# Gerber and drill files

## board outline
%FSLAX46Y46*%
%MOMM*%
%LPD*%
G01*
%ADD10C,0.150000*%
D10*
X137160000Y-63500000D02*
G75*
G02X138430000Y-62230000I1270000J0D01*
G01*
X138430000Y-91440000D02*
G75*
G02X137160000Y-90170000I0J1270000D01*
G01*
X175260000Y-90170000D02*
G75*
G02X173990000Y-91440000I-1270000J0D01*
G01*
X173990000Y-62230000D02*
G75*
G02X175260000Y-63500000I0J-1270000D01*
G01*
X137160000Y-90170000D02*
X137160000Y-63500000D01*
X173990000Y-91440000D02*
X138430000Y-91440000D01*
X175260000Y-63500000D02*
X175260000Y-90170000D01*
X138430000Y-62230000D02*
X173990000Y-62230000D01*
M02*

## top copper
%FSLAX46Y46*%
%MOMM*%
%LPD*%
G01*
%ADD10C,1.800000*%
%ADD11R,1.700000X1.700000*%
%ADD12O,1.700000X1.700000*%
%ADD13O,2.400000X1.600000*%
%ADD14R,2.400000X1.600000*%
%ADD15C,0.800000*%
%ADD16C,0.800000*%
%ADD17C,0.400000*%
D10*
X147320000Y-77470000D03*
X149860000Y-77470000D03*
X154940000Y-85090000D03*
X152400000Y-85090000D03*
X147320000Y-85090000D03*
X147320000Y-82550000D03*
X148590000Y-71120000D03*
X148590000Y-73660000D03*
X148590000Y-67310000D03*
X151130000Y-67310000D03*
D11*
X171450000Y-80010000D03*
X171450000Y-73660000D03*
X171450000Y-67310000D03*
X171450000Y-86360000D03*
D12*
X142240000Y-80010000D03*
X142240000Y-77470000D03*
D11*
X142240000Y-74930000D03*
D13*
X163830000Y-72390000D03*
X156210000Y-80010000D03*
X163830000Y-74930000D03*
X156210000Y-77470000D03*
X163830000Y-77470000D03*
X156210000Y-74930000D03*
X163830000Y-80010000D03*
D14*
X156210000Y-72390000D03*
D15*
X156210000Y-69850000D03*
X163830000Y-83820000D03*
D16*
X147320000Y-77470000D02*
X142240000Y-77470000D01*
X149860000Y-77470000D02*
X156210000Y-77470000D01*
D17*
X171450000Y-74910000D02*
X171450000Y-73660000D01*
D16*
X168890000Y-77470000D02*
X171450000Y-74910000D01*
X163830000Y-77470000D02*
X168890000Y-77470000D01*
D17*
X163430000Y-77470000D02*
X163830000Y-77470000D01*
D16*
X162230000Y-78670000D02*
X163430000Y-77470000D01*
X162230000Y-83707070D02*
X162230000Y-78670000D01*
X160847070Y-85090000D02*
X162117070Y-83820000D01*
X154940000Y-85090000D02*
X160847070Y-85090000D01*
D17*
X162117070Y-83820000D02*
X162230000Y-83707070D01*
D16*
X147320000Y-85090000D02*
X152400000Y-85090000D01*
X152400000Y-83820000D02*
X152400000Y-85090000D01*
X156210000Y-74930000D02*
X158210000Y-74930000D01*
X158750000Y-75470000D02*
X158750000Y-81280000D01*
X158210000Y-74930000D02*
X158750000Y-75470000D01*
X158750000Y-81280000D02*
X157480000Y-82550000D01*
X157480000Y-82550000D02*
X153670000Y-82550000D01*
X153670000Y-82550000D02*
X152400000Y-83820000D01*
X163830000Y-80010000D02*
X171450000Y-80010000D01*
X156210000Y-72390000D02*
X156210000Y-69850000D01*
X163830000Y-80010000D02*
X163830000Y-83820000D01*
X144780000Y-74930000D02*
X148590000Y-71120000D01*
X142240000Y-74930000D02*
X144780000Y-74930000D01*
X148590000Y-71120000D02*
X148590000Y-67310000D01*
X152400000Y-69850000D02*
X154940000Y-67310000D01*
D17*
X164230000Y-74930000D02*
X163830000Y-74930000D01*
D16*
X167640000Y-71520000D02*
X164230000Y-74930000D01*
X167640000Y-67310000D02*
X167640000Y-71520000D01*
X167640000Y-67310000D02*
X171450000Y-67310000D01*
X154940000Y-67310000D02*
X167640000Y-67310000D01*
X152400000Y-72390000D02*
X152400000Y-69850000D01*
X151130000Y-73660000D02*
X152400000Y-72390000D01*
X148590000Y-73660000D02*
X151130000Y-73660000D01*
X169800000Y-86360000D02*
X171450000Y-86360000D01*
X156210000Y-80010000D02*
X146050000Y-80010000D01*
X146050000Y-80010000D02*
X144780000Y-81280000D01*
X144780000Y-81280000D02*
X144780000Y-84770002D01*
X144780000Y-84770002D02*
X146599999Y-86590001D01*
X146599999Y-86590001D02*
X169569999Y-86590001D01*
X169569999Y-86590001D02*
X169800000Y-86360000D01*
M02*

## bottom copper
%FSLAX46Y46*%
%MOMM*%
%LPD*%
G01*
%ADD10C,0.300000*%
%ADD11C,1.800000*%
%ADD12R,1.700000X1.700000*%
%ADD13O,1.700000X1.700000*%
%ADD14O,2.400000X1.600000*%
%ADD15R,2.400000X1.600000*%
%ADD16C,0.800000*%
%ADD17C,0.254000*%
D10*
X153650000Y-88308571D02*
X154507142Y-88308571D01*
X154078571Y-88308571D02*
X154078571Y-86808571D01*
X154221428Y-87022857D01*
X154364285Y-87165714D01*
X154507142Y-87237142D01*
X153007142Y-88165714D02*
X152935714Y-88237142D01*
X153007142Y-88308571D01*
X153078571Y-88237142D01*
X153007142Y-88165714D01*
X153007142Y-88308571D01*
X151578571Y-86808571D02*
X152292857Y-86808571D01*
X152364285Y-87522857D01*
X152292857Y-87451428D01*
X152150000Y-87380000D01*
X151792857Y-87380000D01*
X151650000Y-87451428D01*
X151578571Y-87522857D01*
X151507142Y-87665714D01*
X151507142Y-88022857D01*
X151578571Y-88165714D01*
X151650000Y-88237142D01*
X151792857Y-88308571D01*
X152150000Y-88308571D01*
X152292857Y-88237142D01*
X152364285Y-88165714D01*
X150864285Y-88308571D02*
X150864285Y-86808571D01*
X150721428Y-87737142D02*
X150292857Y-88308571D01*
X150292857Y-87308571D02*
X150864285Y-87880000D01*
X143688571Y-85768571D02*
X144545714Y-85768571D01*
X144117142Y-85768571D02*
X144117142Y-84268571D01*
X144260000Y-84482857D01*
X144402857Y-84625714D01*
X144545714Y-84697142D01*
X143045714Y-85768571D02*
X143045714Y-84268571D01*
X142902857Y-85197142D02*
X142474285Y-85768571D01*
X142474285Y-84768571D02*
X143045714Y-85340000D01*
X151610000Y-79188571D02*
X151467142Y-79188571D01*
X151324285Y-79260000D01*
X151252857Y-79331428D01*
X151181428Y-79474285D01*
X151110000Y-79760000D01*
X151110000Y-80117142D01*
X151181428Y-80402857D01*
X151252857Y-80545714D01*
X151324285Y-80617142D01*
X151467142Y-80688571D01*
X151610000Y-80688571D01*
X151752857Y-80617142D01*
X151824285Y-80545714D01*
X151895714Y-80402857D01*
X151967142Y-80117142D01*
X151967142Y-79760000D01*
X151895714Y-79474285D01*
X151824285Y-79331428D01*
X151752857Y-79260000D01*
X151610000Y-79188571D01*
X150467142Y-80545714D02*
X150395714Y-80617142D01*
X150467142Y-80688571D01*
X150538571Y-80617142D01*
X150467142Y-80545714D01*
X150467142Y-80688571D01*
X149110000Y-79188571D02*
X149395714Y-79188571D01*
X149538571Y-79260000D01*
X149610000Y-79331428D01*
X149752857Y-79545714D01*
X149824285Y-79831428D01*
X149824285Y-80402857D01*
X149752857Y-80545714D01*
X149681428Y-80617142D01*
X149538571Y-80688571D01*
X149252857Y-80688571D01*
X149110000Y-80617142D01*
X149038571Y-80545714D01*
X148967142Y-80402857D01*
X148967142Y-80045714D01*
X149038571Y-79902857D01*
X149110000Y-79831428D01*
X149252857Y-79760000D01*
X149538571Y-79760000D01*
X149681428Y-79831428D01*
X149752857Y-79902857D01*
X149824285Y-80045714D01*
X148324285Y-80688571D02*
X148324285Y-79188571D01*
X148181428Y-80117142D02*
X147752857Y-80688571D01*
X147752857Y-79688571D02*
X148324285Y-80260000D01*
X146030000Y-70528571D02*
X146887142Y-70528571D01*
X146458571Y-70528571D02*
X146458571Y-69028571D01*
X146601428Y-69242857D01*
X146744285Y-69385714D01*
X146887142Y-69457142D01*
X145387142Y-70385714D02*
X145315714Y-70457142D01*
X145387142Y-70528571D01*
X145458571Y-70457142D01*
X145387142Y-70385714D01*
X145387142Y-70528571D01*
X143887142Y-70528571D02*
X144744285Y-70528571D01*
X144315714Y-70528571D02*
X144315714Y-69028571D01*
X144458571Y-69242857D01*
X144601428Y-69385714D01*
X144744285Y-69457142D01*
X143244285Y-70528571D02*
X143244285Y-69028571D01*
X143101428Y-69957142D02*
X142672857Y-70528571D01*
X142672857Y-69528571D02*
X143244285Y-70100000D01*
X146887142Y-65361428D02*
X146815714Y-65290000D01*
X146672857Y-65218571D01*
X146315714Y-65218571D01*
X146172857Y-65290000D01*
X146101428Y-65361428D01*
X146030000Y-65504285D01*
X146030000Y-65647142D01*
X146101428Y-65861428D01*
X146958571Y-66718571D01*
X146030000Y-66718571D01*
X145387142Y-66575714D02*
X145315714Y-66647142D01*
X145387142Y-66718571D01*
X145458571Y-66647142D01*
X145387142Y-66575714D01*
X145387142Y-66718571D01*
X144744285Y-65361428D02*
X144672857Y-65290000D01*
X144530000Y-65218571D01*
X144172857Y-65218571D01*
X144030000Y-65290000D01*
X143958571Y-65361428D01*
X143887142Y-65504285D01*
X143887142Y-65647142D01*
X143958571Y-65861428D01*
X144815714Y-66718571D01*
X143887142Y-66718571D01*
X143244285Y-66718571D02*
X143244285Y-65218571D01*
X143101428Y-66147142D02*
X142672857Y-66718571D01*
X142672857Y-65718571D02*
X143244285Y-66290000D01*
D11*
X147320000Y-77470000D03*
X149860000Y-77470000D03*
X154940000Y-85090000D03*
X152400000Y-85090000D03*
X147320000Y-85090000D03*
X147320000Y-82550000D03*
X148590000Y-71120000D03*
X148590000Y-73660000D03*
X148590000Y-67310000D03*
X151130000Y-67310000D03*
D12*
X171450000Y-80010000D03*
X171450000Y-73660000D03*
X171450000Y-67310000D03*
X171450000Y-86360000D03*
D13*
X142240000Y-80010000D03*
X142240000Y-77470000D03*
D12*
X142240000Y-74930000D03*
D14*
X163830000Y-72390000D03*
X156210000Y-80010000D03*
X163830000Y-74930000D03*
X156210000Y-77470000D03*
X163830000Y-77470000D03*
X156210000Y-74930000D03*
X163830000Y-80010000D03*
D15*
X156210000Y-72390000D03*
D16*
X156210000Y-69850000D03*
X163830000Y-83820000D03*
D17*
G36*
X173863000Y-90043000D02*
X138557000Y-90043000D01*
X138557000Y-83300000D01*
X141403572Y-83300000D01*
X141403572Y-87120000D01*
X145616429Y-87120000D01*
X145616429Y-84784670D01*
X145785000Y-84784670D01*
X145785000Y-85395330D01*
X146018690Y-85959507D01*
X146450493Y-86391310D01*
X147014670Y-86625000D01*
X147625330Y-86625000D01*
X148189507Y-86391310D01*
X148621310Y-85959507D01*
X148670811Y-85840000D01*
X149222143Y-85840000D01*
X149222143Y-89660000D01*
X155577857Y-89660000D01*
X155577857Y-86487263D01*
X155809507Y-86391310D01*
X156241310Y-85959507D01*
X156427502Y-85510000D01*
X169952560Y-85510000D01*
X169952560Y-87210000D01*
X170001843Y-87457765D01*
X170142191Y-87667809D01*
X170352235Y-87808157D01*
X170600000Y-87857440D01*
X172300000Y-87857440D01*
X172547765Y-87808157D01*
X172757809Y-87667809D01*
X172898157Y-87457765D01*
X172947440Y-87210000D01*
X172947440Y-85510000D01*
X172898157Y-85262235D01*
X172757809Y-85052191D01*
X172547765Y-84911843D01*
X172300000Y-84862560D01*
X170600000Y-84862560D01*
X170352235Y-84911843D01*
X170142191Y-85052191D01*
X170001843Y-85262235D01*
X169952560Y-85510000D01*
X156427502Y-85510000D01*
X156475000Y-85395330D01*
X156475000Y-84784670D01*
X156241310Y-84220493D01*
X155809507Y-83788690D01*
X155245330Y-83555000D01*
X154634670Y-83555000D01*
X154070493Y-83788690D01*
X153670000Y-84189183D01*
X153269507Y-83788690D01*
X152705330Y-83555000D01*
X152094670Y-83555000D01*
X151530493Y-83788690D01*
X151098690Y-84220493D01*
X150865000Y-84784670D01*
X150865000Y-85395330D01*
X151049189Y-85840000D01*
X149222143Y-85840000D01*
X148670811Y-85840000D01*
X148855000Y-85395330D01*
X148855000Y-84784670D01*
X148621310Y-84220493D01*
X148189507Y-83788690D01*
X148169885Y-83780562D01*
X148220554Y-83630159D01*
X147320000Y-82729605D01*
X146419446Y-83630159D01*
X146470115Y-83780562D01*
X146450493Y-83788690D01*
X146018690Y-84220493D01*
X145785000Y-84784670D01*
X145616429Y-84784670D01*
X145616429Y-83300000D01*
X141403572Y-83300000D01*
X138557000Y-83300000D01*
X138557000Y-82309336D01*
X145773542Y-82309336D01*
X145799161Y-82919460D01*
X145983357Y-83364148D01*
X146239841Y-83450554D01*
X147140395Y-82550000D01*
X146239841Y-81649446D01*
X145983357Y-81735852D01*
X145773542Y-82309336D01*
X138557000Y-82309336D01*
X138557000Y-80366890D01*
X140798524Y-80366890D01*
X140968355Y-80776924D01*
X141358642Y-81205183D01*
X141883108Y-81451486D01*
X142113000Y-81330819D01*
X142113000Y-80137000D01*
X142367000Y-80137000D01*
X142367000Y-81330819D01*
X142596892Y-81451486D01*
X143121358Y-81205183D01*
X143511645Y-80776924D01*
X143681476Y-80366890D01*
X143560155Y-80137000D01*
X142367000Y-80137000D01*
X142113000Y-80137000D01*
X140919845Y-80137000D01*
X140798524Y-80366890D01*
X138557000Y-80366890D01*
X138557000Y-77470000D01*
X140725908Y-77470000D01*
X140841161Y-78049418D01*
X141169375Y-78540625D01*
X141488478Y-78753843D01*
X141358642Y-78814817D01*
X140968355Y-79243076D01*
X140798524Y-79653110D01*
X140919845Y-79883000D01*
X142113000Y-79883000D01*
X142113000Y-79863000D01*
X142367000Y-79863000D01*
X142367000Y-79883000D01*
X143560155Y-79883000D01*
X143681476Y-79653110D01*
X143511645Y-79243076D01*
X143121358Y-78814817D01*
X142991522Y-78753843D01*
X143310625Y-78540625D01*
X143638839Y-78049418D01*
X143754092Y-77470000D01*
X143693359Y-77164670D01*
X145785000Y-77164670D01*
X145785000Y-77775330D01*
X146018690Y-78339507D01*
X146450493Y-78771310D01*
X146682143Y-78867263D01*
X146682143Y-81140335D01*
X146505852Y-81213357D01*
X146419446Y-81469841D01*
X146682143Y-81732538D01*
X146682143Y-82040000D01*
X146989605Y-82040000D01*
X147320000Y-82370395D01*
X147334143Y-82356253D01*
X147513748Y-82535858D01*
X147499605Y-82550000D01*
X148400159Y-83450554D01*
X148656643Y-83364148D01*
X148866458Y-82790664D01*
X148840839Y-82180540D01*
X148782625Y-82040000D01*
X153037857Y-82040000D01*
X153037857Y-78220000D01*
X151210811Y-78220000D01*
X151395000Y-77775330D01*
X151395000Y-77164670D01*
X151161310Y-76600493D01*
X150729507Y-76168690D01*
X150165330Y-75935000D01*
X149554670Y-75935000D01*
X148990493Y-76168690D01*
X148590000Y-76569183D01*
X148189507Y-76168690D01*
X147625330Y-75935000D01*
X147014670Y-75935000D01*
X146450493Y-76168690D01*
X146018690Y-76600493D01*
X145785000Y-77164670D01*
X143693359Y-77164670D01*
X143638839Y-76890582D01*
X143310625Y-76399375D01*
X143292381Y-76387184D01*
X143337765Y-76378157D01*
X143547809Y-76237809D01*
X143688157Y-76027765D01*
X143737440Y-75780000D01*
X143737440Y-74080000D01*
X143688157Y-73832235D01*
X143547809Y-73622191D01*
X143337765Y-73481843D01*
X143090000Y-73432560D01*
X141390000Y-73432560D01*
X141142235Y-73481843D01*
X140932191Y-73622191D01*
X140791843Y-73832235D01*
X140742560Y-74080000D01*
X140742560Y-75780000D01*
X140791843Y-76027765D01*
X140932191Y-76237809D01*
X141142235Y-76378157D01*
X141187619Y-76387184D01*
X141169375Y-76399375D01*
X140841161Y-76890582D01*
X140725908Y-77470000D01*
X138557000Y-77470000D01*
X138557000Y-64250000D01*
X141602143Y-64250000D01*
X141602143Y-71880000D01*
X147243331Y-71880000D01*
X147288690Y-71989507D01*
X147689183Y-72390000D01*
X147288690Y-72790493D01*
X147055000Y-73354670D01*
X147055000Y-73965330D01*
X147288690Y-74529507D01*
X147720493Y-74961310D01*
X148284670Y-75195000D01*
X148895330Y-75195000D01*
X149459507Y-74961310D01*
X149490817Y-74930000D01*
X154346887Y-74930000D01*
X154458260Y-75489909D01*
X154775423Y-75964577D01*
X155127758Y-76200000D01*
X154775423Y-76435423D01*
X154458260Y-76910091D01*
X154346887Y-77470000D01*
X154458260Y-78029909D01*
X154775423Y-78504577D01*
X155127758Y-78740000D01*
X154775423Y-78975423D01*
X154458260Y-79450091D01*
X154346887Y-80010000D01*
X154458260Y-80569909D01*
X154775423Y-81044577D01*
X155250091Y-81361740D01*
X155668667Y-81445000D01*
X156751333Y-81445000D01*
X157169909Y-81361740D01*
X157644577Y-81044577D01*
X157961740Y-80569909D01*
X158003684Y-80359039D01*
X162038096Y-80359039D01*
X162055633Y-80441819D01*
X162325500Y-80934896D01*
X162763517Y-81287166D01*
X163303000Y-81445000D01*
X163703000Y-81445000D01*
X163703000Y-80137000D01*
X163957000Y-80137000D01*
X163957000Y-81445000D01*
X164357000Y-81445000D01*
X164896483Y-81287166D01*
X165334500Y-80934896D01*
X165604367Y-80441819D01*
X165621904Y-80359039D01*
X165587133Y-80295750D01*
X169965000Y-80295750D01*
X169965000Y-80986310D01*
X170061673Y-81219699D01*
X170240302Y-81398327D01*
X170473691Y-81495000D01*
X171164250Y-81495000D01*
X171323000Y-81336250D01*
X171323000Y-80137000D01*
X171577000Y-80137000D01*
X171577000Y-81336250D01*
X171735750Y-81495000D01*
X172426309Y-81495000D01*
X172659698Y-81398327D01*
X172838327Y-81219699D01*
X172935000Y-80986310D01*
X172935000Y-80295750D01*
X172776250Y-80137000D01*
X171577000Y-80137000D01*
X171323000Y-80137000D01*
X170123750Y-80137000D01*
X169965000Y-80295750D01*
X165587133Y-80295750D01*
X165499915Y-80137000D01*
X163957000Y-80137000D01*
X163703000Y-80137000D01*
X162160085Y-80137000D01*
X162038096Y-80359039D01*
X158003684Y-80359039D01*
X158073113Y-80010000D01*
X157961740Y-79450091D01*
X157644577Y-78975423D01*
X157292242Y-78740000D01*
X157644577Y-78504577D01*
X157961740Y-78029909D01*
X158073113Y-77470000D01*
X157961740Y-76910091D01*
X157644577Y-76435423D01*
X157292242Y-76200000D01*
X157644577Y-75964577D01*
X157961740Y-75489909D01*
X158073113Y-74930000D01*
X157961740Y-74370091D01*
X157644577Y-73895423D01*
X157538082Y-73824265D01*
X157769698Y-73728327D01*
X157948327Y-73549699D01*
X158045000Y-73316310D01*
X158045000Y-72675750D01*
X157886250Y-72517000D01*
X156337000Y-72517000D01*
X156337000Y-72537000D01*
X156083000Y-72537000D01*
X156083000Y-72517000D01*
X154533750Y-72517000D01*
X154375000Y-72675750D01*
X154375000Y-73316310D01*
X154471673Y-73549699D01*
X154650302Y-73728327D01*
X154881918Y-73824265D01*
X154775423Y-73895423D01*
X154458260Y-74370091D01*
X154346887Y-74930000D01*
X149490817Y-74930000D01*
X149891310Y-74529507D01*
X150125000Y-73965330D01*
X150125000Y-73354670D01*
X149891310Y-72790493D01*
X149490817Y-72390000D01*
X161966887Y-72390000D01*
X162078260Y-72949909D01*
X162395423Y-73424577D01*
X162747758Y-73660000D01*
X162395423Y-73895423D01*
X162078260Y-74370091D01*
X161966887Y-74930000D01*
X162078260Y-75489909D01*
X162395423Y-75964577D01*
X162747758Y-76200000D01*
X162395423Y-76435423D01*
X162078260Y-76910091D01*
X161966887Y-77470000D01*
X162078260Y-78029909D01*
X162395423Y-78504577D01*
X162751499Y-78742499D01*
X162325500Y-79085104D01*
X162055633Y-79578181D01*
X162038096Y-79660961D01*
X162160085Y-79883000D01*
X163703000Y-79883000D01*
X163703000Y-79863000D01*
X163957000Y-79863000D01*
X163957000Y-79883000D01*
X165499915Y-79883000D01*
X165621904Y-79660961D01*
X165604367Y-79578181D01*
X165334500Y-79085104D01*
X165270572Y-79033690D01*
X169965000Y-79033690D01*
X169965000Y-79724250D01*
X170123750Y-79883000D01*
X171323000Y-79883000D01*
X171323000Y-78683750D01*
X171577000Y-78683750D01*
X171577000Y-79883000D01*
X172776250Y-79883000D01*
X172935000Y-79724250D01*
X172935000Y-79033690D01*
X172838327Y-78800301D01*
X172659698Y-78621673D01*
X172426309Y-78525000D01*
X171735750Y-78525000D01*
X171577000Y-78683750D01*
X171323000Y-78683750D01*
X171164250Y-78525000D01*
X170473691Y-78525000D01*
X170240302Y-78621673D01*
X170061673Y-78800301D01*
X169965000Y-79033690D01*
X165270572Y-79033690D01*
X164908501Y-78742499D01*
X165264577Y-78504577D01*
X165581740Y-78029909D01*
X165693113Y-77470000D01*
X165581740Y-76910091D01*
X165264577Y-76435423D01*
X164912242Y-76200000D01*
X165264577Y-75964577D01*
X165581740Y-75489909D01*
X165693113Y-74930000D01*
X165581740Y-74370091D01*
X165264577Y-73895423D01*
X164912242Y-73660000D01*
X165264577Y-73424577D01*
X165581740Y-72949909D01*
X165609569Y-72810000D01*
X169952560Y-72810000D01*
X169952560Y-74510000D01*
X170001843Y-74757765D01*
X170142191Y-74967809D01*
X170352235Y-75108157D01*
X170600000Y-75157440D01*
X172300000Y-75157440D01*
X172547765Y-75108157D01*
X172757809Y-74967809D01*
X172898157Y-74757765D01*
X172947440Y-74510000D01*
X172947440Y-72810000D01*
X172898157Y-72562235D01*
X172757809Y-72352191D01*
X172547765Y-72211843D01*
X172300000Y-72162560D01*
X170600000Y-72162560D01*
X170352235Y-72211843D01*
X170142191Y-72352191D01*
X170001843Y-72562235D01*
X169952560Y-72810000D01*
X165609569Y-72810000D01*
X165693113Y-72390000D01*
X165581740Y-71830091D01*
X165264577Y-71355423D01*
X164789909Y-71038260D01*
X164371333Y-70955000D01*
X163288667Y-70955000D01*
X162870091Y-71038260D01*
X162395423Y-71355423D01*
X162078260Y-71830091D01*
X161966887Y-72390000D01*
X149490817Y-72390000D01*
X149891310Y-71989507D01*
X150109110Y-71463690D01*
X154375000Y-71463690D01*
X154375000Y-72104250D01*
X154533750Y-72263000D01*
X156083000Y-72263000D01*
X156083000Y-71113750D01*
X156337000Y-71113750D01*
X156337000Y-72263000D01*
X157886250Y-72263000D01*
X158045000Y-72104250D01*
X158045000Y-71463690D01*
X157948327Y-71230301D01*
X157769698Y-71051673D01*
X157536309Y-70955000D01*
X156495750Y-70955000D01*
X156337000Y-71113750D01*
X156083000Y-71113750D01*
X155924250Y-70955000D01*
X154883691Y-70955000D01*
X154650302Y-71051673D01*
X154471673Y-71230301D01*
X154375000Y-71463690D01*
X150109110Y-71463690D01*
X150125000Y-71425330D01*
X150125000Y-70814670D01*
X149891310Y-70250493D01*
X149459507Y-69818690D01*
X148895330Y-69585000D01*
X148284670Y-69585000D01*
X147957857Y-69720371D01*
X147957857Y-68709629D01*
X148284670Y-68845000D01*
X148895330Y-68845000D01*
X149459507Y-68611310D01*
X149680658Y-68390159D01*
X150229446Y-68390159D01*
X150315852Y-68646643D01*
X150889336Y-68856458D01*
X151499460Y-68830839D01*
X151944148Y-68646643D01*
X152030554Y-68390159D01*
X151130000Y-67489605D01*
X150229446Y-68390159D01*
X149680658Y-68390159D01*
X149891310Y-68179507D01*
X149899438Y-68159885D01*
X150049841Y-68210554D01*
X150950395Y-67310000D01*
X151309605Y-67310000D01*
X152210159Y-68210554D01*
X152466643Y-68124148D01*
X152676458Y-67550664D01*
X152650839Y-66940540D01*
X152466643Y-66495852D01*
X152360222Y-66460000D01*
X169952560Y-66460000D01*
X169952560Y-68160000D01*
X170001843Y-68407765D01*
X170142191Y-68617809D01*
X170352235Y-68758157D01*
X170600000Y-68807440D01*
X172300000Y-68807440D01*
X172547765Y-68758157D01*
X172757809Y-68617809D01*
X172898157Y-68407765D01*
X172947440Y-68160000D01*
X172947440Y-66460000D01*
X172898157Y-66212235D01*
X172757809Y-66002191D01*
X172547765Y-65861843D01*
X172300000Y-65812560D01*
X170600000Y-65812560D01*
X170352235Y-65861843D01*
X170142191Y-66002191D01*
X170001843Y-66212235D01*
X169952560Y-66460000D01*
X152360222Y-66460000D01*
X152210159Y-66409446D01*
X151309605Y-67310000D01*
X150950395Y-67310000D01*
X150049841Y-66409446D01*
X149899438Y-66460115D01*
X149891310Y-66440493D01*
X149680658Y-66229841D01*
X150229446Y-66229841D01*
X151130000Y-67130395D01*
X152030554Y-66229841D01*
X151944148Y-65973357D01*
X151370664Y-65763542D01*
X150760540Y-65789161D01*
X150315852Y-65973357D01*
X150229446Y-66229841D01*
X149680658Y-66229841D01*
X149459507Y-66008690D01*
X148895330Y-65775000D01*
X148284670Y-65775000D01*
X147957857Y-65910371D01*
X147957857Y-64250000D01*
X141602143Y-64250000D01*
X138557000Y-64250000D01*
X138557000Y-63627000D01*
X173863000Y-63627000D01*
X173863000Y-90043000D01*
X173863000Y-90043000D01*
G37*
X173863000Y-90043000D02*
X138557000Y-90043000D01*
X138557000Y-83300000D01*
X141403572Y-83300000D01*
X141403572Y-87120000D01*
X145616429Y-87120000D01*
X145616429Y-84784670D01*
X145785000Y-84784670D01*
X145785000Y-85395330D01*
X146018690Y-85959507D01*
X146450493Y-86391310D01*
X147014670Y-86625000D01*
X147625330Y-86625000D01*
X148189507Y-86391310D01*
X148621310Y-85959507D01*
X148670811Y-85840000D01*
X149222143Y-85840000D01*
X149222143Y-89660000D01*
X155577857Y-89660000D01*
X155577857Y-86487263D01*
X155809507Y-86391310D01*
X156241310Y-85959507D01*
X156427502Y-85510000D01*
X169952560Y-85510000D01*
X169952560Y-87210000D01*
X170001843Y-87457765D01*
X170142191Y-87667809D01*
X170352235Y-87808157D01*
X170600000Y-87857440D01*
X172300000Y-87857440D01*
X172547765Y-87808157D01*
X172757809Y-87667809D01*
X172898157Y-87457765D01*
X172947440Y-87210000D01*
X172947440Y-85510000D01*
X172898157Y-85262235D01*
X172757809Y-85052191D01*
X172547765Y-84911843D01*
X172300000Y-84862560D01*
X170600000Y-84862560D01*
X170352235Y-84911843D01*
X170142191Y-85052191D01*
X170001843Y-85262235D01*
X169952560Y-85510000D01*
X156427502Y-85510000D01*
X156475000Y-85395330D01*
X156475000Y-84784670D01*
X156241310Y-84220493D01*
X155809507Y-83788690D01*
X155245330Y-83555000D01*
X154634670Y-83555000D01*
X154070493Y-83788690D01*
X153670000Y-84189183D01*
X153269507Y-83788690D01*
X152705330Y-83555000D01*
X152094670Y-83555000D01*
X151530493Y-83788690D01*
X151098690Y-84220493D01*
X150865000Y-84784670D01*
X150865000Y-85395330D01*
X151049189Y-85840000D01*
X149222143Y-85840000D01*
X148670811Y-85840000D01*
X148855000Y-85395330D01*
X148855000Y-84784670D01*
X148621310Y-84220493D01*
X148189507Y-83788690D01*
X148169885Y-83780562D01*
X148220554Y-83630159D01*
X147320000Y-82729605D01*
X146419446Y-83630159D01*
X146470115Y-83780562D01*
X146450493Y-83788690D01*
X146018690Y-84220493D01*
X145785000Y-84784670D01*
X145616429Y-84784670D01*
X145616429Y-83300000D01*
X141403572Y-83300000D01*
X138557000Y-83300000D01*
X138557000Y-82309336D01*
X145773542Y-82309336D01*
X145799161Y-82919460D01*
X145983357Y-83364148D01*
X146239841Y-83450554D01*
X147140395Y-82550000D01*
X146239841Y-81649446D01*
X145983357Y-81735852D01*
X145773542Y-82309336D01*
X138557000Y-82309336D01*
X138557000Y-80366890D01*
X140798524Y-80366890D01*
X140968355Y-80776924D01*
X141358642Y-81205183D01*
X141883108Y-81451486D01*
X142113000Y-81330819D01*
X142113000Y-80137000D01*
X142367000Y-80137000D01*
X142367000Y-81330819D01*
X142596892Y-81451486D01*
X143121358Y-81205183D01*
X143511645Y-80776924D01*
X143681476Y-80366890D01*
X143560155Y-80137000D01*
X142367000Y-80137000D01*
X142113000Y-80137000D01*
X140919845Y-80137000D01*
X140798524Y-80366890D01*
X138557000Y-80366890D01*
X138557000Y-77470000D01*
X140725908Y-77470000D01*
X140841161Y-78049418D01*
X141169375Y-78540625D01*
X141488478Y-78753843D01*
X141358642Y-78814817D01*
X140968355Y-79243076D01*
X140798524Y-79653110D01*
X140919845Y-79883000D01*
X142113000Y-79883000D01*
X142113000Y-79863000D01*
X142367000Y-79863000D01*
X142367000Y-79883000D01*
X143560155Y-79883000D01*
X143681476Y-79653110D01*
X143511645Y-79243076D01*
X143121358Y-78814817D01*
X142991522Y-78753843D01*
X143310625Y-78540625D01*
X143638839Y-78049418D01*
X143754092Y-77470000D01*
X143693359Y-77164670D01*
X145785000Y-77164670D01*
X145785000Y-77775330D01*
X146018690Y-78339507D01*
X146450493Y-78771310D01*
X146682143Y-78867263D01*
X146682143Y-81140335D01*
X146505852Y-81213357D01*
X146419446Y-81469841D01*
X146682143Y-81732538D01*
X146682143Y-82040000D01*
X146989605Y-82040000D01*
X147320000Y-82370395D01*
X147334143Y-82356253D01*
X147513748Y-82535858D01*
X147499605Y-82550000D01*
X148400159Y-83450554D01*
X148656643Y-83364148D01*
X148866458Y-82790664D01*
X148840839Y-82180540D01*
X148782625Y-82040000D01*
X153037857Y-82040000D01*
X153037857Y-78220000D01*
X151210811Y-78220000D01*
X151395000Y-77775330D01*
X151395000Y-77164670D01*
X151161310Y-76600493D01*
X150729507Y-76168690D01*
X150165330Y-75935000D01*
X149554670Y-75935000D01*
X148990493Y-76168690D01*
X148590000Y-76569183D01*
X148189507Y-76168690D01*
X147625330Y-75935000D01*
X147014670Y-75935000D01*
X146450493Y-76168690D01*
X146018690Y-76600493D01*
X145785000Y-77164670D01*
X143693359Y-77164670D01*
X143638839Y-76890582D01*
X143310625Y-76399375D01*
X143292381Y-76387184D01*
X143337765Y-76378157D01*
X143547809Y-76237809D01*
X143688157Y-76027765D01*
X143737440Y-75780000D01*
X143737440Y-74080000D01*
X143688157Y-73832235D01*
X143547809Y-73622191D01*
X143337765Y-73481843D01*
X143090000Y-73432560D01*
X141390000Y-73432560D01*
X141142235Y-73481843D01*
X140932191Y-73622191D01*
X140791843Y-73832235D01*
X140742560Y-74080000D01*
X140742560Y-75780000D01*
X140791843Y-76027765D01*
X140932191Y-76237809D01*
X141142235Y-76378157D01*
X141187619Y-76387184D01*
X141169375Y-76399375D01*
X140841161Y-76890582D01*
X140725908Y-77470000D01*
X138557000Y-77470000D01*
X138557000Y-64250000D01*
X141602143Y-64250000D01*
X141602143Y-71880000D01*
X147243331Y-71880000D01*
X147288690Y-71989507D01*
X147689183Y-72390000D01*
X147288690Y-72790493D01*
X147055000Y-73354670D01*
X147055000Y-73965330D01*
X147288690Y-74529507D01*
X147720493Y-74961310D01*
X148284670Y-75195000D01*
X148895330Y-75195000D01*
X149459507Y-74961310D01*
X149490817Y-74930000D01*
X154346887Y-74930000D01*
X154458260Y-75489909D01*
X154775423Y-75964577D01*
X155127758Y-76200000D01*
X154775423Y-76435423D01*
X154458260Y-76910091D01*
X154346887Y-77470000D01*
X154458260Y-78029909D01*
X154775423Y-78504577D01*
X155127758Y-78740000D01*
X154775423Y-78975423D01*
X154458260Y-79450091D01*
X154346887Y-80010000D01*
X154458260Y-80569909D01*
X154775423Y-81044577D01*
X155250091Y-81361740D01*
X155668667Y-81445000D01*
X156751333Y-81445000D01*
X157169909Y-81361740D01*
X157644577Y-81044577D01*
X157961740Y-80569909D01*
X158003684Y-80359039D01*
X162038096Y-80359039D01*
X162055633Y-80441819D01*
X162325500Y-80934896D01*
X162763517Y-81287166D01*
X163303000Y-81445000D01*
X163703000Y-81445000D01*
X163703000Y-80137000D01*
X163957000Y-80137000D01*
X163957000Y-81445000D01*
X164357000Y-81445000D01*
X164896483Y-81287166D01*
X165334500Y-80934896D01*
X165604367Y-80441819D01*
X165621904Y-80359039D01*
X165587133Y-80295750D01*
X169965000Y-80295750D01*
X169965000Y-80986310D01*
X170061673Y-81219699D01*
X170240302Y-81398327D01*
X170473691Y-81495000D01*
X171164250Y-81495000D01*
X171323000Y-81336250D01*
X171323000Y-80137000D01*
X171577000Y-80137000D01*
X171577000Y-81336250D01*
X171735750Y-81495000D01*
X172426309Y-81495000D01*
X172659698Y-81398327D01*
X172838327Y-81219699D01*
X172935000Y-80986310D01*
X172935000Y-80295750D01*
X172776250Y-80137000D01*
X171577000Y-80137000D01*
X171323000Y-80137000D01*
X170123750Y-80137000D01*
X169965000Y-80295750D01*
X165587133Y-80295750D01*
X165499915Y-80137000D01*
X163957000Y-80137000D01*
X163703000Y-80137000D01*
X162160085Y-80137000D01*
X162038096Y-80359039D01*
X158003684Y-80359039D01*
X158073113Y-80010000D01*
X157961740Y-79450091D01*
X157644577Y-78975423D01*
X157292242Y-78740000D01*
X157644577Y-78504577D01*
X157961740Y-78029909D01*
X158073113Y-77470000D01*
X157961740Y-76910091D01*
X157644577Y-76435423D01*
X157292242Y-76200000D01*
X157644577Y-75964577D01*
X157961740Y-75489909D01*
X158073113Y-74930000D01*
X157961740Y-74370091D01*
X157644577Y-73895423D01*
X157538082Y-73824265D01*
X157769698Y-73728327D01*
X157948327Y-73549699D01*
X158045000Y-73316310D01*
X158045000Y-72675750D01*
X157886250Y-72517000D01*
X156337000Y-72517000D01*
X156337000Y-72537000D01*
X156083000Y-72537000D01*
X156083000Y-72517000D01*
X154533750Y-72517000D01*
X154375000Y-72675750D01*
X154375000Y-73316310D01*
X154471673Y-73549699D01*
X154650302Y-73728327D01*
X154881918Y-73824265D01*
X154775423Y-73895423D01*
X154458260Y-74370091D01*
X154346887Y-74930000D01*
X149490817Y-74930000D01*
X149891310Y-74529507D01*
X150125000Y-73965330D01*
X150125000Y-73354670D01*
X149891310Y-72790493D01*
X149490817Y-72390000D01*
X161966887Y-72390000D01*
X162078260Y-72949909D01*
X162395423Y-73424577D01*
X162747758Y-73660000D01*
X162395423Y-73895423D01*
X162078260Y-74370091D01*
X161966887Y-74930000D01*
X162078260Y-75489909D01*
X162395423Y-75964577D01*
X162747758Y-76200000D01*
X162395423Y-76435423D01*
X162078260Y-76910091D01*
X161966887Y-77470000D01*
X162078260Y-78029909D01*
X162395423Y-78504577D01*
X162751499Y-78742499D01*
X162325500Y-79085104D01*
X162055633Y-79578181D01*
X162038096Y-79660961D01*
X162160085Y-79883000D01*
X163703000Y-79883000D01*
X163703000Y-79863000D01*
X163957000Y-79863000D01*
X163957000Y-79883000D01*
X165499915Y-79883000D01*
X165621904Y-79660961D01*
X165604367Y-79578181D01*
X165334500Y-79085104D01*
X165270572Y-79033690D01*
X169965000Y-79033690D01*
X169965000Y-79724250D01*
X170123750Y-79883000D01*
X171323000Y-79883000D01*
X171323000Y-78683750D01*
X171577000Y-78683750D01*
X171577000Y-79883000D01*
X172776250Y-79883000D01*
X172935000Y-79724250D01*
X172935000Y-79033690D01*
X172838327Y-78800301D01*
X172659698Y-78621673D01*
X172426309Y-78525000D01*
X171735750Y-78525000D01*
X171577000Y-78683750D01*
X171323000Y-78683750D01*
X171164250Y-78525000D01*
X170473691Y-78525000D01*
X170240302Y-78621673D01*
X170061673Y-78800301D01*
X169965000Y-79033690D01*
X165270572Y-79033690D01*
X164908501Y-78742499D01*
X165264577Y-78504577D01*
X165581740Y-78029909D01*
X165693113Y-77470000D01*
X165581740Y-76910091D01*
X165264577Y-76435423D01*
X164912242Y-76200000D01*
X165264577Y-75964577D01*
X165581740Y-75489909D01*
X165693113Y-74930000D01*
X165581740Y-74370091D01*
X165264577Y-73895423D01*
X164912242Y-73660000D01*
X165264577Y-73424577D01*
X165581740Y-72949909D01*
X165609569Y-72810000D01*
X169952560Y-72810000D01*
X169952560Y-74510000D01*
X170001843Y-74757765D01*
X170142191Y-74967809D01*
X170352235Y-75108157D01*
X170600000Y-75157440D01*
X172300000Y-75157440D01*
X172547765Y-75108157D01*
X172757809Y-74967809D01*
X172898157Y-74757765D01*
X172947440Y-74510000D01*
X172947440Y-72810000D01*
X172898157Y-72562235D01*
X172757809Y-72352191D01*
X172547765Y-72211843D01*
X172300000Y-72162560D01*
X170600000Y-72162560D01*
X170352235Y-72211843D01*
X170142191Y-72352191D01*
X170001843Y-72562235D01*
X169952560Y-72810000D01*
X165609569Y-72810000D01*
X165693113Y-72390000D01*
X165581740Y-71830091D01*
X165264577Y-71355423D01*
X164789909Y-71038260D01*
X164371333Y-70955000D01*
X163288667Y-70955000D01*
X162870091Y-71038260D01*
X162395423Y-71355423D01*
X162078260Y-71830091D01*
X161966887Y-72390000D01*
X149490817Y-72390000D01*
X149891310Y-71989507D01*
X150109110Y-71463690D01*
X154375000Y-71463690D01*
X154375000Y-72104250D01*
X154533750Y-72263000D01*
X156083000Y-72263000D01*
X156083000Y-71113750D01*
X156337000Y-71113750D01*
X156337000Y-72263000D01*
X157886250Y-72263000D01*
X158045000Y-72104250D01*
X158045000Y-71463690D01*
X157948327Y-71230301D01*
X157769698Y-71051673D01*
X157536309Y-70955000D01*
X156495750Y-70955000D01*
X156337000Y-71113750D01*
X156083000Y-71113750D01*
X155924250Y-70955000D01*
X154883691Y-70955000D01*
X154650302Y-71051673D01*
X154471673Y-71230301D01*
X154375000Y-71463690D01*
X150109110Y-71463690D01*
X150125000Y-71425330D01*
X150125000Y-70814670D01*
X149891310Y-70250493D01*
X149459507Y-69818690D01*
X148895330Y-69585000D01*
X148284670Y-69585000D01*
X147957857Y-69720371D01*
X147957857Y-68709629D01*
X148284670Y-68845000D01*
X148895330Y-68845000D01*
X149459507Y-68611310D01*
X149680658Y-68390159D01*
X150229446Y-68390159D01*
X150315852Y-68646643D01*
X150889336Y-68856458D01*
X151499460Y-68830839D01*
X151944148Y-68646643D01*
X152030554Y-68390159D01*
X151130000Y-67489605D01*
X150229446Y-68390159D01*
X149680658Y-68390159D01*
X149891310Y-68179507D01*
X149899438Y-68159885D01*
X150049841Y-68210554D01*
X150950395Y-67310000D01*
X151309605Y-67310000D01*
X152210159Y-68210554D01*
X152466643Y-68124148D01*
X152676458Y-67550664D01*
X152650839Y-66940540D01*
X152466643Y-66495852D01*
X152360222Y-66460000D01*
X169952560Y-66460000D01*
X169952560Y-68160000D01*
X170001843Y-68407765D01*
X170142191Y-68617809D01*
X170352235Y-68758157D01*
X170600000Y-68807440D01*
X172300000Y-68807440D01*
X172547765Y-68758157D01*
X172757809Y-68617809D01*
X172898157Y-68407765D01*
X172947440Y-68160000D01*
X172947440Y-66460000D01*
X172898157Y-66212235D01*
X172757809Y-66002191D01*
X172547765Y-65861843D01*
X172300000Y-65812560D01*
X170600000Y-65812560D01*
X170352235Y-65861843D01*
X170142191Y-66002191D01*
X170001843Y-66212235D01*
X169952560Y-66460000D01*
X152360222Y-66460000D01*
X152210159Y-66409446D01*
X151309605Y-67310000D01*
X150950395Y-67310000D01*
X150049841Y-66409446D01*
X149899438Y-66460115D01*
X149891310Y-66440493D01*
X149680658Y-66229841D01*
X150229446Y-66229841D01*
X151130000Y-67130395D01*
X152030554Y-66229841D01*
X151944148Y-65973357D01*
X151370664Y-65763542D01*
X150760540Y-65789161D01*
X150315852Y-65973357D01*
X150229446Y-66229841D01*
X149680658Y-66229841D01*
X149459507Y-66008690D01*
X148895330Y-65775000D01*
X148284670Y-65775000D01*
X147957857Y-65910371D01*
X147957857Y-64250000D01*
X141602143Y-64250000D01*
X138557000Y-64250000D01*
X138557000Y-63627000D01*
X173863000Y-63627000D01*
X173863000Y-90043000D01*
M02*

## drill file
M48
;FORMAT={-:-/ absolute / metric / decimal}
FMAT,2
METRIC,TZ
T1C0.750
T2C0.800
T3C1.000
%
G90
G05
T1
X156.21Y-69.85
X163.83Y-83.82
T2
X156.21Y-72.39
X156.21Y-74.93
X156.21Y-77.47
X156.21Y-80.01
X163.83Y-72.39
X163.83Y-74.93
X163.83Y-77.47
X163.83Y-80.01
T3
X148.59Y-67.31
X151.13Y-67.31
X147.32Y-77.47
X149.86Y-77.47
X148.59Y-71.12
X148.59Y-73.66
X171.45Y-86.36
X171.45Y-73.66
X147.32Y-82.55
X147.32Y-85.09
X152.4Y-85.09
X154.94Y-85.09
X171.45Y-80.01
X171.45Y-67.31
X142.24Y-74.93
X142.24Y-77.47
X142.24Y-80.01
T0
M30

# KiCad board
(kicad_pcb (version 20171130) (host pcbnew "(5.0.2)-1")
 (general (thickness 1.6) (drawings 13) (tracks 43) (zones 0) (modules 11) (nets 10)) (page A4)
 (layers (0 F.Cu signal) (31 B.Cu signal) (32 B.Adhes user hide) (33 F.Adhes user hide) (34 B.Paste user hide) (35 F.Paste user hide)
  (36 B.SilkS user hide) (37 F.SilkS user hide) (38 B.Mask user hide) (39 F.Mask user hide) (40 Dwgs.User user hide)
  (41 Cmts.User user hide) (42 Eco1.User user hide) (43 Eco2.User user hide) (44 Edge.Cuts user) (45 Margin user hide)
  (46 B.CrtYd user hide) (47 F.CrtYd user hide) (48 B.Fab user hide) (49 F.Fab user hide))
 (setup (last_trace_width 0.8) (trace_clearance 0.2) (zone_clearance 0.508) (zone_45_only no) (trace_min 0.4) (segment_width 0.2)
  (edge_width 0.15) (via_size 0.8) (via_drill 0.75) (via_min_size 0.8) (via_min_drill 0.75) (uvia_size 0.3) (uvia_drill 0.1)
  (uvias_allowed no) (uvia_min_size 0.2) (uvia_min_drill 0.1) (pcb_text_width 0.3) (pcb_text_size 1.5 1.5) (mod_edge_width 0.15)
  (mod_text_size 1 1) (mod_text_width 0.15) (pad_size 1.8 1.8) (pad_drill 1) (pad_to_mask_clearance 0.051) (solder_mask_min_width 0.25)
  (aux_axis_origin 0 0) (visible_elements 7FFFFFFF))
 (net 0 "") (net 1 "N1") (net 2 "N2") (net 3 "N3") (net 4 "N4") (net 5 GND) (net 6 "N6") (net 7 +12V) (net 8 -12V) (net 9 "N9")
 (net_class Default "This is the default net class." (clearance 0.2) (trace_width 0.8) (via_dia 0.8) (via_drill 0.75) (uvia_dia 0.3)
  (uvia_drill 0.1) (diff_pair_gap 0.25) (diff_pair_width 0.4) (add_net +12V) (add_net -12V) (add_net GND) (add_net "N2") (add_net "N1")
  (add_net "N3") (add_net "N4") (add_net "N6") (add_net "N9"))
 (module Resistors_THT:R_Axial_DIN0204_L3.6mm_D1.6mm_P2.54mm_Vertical (layer F.Cu) (at 149.86 77.47 180)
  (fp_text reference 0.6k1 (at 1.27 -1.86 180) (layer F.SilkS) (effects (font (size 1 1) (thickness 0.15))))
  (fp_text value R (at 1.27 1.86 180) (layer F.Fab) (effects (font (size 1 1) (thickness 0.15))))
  (pad 2 thru_hole circle (at 2.54 0 180) (size 1.8 1.8) (drill 1) (layers *.Cu *.Mask) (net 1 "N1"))
  (pad 1 thru_hole circle (at 0 0 180) (size 1.8 1.8) (drill 1) (layers *.Cu *.Mask) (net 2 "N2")))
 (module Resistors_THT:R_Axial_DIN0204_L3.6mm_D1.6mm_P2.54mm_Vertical (layer F.Cu) (at 154.94 85.09 180)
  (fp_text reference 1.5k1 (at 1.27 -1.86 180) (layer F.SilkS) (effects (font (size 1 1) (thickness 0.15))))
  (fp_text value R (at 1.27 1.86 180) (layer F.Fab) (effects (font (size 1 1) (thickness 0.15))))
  (pad e thru_hole circle (at 0 0 180) (size 1.8 1.8) (drill 1) (layers *.Cu *.Mask) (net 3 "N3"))
  (pad 2 thru_hole circle (at 2.54 0 180) (size 1.8 1.8) (drill 1) (layers *.Cu *.Mask) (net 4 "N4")))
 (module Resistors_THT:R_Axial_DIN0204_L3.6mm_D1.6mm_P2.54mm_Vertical (layer F.Cu) (at 147.32 82.55 270)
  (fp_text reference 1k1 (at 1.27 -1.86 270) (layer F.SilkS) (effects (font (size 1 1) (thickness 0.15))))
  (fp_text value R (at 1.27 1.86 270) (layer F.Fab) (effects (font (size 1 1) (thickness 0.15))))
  (pad 2 thru_hole circle (at 2.54 0 270) (size 1.8 1.8) (drill 1) (layers *.Cu *.Mask) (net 4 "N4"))
  (pad 1 thru_hole circle (at 0 0 270) (size 1.8 1.8) (drill 1) (layers *.Cu *.Mask) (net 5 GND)))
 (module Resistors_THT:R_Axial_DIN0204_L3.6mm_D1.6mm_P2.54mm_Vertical (layer F.Cu) (at 148.59 73.66 90)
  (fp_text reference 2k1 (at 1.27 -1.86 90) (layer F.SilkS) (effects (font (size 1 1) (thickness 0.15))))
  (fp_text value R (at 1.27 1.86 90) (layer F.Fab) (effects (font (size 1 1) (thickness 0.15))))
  (pad 2 thru_hole circle (at 2.54 0 90) (size 1.8 1.8) (drill 1) (layers *.Cu *.Mask) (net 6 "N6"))
  (pad 1 thru_hole circle (at 0 0 90) (size 1.8 1.8) (drill 1) (layers *.Cu *.Mask) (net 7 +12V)))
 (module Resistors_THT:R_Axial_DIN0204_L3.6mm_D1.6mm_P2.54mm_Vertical (layer F.Cu) (at 148.59 67.31)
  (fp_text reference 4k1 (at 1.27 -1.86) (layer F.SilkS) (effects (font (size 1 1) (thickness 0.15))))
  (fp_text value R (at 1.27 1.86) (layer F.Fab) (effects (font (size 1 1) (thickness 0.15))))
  (pad e thru_hole circle (at 0 0) (size 1.8 1.8) (drill 1) (layers *.Cu *.Mask) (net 6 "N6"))
  (pad 2 thru_hole circle (at 2.54 0) (size 1.8 1.8) (drill 1) (layers *.Cu *.Mask) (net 5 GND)))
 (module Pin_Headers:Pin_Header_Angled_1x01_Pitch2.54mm (layer F.Cu) (at 171.45 80.01)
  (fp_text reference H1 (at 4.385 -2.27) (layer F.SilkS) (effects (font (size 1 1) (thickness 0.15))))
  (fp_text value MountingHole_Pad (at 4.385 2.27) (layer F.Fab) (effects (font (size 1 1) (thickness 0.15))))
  (pad 1 thru_hole rect (at 0 0) (size 1.7 1.7) (drill 1) (layers *.Cu *.Mask) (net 5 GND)))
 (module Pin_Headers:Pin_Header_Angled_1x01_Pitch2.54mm (layer F.Cu) (at 171.45 73.66)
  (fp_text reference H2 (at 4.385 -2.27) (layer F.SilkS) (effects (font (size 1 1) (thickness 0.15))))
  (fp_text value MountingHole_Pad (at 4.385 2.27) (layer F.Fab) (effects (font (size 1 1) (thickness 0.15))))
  (pad 1 thru_hole rect (at 0 0) (size 1.7 1.7) (drill 1) (layers *.Cu *.Mask) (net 3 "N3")))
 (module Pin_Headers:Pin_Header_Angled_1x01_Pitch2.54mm (layer F.Cu) (at 171.45 67.31)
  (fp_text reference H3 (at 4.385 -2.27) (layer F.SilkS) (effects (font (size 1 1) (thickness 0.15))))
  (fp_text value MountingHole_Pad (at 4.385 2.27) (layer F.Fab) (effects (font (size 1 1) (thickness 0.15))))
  (pad 1 thru_hole rect (at 0 0) (size 1.7 1.7) (drill 1) (layers *.Cu *.Mask) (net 7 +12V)))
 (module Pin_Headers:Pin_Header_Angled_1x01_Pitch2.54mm (layer F.Cu) (at 171.45 86.36)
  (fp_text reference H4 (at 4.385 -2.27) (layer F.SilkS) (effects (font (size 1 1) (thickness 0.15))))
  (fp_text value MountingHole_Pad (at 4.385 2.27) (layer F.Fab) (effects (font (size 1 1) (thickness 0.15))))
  (pad 1 thru_hole rect (at 0 0) (size 1.7 1.7) (drill 1) (layers *.Cu *.Mask) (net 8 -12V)))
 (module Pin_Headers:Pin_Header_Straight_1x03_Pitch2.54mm (layer F.Cu) (at 142.24 74.93)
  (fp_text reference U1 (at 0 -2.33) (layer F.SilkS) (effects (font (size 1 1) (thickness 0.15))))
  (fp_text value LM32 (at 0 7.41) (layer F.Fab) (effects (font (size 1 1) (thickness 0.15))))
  (pad 3 thru_hole oval (at 0 5.08) (size 1.7 1.7) (drill 1) (layers *.Cu *.Mask) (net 5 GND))
  (pad 2 thru_hole oval (at 0 2.54) (size 1.7 1.7) (drill 1) (layers *.Cu *.Mask) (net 1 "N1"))
  (pad 1 thru_hole rect (at 0 0) (size 1.7 1.7) (drill 1) (layers *.Cu *.Mask) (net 6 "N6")))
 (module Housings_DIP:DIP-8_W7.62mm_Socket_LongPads (layer F.Cu) (at 156.21 72.39)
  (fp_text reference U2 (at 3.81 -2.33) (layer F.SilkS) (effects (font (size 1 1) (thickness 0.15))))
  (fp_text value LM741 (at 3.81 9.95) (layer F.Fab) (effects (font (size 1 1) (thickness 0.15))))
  (pad 8 thru_hole oval (at 7.62 0) (size 2.4 1.6) (drill 0.8) (layers *.Cu *.Mask) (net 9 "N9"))
  (pad 4 thru_hole oval (at 0 7.62) (size 2.4 1.6) (drill 0.8) (layers *.Cu *.Mask) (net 8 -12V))
  (pad 7 thru_hole oval (at 7.62 2.54) (size 2.4 1.6) (drill 0.8) (layers *.Cu *.Mask) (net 7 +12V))
  (pad 3 thru_hole oval (at 0 5.08) (size 2.4 1.6) (drill 0.8) (layers *.Cu *.Mask) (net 2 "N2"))
  (pad 6 thru_hole oval (at 7.62 5.08) (size 2.4 1.6) (drill 0.8) (layers *.Cu *.Mask) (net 3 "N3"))
  (pad 2 thru_hole oval (at 0 2.54) (size 2.4 1.6) (drill 0.8) (layers *.Cu *.Mask) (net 4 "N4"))
  (pad 5 thru_hole oval (at 7.62 7.62) (size 2.4 1.6) (drill 0.8) (layers *.Cu *.Mask) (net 5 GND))
  (pad 1 thru_hole rect (at 0 0) (size 2.4 1.6) (drill 0.8) (layers *.Cu *.Mask) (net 5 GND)))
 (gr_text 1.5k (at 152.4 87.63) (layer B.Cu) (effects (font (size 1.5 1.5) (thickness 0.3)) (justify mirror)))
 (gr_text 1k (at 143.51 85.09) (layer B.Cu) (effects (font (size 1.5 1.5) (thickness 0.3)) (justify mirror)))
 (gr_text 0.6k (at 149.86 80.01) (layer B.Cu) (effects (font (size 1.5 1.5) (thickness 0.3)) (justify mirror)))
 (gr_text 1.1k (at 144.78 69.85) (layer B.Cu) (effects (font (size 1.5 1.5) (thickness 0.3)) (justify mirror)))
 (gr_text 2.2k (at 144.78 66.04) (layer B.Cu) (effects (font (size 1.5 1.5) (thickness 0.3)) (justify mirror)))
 (gr_arc (start 138.43 63.5) (end 138.43 62.23) (angle -90) (layer Edge.Cuts) (width 0.15))
 (gr_arc (start 138.43 90.17) (end 137.16 90.17) (angle -90) (layer Edge.Cuts) (width 0.15))
 (gr_arc (start 173.99 90.17) (end 173.99 91.44) (angle -90) (layer Edge.Cuts) (width 0.15))
 (gr_arc (start 173.99 63.5) (end 175.26 63.5) (angle -90) (layer Edge.Cuts) (width 0.15))
 (gr_line (start 137.16 90.17) (end 137.16 63.5) (layer Edge.Cuts) (width 0.15))
 (gr_line (start 173.99 91.44) (end 138.43 91.44) (layer Edge.Cuts) (width 0.15))
 (gr_line (start 175.26 63.5) (end 175.26 90.17) (layer Edge.Cuts) (width 0.15))
 (gr_line (start 138.43 62.23) (end 173.99 62.23) (layer Edge.Cuts) (width 0.15))
 (segment (start 147.32 77.47) (end 142.24 77.47) (width 0.8) (layer F.Cu) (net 1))
 (segment (start 149.86 77.47) (end 156.21 77.47) (width 0.8) (layer F.Cu) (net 2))
 (segment (start 171.45 74.91) (end 171.45 73.66) (width 0.4) (layer F.Cu) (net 3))
 (segment (start 168.89 77.47) (end 171.45 74.91) (width 0.8) (layer F.Cu) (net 3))
 (segment (start 163.83 77.47) (end 168.89 77.47) (width 0.8) (layer F.Cu) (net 3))
 (segment (start 163.43 77.47) (end 163.83 77.47) (width 0.4) (layer F.Cu) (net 3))
 (segment (start 162.23 78.67) (end 163.43 77.47) (width 0.8) (layer F.Cu) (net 3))
 (segment (start 162.23 83.70707) (end 162.23 78.67) (width 0.8) (layer F.Cu) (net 3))
 (segment (start 160.84707 85.09) (end 162.11707 83.82) (width 0.8) (layer F.Cu) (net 3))
 (segment (start 154.94 85.09) (end 160.84707 85.09) (width 0.8) (layer F.Cu) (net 3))
 (segment (start 162.11707 83.82) (end 162.23 83.70707) (width 0.4) (layer F.Cu) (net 3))
 (segment (start 147.32 85.09) (end 152.4 85.09) (width 0.8) (layer F.Cu) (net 4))
 (segment (start 152.4 83.82) (end 152.4 85.09) (width 0.8) (layer F.Cu) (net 4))
 (segment (start 156.21 74.93) (end 158.21 74.93) (width 0.8) (layer F.Cu) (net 4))
 (segment (start 158.75 75.47) (end 158.75 81.28) (width 0.8) (layer F.Cu) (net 4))
 (segment (start 158.21 74.93) (end 158.75 75.47) (width 0.8) (layer F.Cu) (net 4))
 (segment (start 158.75 81.28) (end 157.48 82.55) (width 0.8) (layer F.Cu) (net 4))
 (segment (start 157.48 82.55) (end 153.67 82.55) (width 0.8) (layer F.Cu) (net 4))
 (segment (start 153.67 82.55) (end 152.4 83.82) (width 0.8) (layer F.Cu) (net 4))
 (segment (start 163.83 80.01) (end 171.45 80.01) (width 0.8) (layer F.Cu) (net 5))
 (segment (start 156.21 72.39) (end 156.21 69.85) (width 0.8) (layer F.Cu) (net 5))
 (via (at 156.21 69.85) (size 0.8) (drill 0.75) (layers F.Cu B.Cu) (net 5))
 (segment (start 163.83 80.01) (end 163.83 83.82) (width 0.8) (layer F.Cu) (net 5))
 (via (at 163.83 83.82) (size 0.8) (drill 0.75) (layers F.Cu B.Cu) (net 5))
 (segment (start 144.78 74.93) (end 148.59 71.12) (width 0.8) (layer F.Cu) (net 6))
 (segment (start 142.24 74.93) (end 144.78 74.93) (width 0.8) (layer F.Cu) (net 6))
 (segment (start 148.59 71.12) (end 148.59 67.31) (width 0.8) (layer F.Cu) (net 6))
 (segment (start 152.4 69.85) (end 154.94 67.31) (width 0.8) (layer F.Cu) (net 7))
 (segment (start 164.23 74.93) (end 163.83 74.93) (width 0.4) (layer F.Cu) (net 7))
 (segment (start 167.64 71.52) (end 164.23 74.93) (width 0.8) (layer F.Cu) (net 7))
 (segment (start 167.64 67.31) (end 167.64 71.52) (width 0.8) (layer F.Cu) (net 7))
 (segment (start 167.64 67.31) (end 171.45 67.31) (width 0.8) (layer F.Cu) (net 7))
 (segment (start 154.94 67.31) (end 167.64 67.31) (width 0.8) (layer F.Cu) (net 7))
 (segment (start 152.4 72.39) (end 152.4 69.85) (width 0.8) (layer F.Cu) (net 7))
 (segment (start 151.13 73.66) (end 152.4 72.39) (width 0.8) (layer F.Cu) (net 7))
 (segment (start 148.59 73.66) (end 151.13 73.66) (width 0.8) (layer F.Cu) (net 7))
 (segment (start 169.8 86.36) (end 171.45 86.36) (width 0.8) (layer F.Cu) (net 8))
 (segment (start 156.21 80.01) (end 146.05 80.01) (width 0.8) (layer F.Cu) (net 8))
 (segment (start 146.05 80.01) (end 144.78 81.28) (width 0.8) (layer F.Cu) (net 8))
 (segment (start 144.78 81.28) (end 144.78 84.770002) (width 0.8) (layer F.Cu) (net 8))
 (segment (start 144.78 84.770002) (end 146.599999 86.590001) (width 0.8) (layer F.Cu) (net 8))
 (segment (start 146.599999 86.590001) (end 169.569999 86.590001) (width 0.8) (layer F.Cu) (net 8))
 (segment (start 169.569999 86.590001) (end 169.8 86.36) (width 0.8) (layer F.Cu) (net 8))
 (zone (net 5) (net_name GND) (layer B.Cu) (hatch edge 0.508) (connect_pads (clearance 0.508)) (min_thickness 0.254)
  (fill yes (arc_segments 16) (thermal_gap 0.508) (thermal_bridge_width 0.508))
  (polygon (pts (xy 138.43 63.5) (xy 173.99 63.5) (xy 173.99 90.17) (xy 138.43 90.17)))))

